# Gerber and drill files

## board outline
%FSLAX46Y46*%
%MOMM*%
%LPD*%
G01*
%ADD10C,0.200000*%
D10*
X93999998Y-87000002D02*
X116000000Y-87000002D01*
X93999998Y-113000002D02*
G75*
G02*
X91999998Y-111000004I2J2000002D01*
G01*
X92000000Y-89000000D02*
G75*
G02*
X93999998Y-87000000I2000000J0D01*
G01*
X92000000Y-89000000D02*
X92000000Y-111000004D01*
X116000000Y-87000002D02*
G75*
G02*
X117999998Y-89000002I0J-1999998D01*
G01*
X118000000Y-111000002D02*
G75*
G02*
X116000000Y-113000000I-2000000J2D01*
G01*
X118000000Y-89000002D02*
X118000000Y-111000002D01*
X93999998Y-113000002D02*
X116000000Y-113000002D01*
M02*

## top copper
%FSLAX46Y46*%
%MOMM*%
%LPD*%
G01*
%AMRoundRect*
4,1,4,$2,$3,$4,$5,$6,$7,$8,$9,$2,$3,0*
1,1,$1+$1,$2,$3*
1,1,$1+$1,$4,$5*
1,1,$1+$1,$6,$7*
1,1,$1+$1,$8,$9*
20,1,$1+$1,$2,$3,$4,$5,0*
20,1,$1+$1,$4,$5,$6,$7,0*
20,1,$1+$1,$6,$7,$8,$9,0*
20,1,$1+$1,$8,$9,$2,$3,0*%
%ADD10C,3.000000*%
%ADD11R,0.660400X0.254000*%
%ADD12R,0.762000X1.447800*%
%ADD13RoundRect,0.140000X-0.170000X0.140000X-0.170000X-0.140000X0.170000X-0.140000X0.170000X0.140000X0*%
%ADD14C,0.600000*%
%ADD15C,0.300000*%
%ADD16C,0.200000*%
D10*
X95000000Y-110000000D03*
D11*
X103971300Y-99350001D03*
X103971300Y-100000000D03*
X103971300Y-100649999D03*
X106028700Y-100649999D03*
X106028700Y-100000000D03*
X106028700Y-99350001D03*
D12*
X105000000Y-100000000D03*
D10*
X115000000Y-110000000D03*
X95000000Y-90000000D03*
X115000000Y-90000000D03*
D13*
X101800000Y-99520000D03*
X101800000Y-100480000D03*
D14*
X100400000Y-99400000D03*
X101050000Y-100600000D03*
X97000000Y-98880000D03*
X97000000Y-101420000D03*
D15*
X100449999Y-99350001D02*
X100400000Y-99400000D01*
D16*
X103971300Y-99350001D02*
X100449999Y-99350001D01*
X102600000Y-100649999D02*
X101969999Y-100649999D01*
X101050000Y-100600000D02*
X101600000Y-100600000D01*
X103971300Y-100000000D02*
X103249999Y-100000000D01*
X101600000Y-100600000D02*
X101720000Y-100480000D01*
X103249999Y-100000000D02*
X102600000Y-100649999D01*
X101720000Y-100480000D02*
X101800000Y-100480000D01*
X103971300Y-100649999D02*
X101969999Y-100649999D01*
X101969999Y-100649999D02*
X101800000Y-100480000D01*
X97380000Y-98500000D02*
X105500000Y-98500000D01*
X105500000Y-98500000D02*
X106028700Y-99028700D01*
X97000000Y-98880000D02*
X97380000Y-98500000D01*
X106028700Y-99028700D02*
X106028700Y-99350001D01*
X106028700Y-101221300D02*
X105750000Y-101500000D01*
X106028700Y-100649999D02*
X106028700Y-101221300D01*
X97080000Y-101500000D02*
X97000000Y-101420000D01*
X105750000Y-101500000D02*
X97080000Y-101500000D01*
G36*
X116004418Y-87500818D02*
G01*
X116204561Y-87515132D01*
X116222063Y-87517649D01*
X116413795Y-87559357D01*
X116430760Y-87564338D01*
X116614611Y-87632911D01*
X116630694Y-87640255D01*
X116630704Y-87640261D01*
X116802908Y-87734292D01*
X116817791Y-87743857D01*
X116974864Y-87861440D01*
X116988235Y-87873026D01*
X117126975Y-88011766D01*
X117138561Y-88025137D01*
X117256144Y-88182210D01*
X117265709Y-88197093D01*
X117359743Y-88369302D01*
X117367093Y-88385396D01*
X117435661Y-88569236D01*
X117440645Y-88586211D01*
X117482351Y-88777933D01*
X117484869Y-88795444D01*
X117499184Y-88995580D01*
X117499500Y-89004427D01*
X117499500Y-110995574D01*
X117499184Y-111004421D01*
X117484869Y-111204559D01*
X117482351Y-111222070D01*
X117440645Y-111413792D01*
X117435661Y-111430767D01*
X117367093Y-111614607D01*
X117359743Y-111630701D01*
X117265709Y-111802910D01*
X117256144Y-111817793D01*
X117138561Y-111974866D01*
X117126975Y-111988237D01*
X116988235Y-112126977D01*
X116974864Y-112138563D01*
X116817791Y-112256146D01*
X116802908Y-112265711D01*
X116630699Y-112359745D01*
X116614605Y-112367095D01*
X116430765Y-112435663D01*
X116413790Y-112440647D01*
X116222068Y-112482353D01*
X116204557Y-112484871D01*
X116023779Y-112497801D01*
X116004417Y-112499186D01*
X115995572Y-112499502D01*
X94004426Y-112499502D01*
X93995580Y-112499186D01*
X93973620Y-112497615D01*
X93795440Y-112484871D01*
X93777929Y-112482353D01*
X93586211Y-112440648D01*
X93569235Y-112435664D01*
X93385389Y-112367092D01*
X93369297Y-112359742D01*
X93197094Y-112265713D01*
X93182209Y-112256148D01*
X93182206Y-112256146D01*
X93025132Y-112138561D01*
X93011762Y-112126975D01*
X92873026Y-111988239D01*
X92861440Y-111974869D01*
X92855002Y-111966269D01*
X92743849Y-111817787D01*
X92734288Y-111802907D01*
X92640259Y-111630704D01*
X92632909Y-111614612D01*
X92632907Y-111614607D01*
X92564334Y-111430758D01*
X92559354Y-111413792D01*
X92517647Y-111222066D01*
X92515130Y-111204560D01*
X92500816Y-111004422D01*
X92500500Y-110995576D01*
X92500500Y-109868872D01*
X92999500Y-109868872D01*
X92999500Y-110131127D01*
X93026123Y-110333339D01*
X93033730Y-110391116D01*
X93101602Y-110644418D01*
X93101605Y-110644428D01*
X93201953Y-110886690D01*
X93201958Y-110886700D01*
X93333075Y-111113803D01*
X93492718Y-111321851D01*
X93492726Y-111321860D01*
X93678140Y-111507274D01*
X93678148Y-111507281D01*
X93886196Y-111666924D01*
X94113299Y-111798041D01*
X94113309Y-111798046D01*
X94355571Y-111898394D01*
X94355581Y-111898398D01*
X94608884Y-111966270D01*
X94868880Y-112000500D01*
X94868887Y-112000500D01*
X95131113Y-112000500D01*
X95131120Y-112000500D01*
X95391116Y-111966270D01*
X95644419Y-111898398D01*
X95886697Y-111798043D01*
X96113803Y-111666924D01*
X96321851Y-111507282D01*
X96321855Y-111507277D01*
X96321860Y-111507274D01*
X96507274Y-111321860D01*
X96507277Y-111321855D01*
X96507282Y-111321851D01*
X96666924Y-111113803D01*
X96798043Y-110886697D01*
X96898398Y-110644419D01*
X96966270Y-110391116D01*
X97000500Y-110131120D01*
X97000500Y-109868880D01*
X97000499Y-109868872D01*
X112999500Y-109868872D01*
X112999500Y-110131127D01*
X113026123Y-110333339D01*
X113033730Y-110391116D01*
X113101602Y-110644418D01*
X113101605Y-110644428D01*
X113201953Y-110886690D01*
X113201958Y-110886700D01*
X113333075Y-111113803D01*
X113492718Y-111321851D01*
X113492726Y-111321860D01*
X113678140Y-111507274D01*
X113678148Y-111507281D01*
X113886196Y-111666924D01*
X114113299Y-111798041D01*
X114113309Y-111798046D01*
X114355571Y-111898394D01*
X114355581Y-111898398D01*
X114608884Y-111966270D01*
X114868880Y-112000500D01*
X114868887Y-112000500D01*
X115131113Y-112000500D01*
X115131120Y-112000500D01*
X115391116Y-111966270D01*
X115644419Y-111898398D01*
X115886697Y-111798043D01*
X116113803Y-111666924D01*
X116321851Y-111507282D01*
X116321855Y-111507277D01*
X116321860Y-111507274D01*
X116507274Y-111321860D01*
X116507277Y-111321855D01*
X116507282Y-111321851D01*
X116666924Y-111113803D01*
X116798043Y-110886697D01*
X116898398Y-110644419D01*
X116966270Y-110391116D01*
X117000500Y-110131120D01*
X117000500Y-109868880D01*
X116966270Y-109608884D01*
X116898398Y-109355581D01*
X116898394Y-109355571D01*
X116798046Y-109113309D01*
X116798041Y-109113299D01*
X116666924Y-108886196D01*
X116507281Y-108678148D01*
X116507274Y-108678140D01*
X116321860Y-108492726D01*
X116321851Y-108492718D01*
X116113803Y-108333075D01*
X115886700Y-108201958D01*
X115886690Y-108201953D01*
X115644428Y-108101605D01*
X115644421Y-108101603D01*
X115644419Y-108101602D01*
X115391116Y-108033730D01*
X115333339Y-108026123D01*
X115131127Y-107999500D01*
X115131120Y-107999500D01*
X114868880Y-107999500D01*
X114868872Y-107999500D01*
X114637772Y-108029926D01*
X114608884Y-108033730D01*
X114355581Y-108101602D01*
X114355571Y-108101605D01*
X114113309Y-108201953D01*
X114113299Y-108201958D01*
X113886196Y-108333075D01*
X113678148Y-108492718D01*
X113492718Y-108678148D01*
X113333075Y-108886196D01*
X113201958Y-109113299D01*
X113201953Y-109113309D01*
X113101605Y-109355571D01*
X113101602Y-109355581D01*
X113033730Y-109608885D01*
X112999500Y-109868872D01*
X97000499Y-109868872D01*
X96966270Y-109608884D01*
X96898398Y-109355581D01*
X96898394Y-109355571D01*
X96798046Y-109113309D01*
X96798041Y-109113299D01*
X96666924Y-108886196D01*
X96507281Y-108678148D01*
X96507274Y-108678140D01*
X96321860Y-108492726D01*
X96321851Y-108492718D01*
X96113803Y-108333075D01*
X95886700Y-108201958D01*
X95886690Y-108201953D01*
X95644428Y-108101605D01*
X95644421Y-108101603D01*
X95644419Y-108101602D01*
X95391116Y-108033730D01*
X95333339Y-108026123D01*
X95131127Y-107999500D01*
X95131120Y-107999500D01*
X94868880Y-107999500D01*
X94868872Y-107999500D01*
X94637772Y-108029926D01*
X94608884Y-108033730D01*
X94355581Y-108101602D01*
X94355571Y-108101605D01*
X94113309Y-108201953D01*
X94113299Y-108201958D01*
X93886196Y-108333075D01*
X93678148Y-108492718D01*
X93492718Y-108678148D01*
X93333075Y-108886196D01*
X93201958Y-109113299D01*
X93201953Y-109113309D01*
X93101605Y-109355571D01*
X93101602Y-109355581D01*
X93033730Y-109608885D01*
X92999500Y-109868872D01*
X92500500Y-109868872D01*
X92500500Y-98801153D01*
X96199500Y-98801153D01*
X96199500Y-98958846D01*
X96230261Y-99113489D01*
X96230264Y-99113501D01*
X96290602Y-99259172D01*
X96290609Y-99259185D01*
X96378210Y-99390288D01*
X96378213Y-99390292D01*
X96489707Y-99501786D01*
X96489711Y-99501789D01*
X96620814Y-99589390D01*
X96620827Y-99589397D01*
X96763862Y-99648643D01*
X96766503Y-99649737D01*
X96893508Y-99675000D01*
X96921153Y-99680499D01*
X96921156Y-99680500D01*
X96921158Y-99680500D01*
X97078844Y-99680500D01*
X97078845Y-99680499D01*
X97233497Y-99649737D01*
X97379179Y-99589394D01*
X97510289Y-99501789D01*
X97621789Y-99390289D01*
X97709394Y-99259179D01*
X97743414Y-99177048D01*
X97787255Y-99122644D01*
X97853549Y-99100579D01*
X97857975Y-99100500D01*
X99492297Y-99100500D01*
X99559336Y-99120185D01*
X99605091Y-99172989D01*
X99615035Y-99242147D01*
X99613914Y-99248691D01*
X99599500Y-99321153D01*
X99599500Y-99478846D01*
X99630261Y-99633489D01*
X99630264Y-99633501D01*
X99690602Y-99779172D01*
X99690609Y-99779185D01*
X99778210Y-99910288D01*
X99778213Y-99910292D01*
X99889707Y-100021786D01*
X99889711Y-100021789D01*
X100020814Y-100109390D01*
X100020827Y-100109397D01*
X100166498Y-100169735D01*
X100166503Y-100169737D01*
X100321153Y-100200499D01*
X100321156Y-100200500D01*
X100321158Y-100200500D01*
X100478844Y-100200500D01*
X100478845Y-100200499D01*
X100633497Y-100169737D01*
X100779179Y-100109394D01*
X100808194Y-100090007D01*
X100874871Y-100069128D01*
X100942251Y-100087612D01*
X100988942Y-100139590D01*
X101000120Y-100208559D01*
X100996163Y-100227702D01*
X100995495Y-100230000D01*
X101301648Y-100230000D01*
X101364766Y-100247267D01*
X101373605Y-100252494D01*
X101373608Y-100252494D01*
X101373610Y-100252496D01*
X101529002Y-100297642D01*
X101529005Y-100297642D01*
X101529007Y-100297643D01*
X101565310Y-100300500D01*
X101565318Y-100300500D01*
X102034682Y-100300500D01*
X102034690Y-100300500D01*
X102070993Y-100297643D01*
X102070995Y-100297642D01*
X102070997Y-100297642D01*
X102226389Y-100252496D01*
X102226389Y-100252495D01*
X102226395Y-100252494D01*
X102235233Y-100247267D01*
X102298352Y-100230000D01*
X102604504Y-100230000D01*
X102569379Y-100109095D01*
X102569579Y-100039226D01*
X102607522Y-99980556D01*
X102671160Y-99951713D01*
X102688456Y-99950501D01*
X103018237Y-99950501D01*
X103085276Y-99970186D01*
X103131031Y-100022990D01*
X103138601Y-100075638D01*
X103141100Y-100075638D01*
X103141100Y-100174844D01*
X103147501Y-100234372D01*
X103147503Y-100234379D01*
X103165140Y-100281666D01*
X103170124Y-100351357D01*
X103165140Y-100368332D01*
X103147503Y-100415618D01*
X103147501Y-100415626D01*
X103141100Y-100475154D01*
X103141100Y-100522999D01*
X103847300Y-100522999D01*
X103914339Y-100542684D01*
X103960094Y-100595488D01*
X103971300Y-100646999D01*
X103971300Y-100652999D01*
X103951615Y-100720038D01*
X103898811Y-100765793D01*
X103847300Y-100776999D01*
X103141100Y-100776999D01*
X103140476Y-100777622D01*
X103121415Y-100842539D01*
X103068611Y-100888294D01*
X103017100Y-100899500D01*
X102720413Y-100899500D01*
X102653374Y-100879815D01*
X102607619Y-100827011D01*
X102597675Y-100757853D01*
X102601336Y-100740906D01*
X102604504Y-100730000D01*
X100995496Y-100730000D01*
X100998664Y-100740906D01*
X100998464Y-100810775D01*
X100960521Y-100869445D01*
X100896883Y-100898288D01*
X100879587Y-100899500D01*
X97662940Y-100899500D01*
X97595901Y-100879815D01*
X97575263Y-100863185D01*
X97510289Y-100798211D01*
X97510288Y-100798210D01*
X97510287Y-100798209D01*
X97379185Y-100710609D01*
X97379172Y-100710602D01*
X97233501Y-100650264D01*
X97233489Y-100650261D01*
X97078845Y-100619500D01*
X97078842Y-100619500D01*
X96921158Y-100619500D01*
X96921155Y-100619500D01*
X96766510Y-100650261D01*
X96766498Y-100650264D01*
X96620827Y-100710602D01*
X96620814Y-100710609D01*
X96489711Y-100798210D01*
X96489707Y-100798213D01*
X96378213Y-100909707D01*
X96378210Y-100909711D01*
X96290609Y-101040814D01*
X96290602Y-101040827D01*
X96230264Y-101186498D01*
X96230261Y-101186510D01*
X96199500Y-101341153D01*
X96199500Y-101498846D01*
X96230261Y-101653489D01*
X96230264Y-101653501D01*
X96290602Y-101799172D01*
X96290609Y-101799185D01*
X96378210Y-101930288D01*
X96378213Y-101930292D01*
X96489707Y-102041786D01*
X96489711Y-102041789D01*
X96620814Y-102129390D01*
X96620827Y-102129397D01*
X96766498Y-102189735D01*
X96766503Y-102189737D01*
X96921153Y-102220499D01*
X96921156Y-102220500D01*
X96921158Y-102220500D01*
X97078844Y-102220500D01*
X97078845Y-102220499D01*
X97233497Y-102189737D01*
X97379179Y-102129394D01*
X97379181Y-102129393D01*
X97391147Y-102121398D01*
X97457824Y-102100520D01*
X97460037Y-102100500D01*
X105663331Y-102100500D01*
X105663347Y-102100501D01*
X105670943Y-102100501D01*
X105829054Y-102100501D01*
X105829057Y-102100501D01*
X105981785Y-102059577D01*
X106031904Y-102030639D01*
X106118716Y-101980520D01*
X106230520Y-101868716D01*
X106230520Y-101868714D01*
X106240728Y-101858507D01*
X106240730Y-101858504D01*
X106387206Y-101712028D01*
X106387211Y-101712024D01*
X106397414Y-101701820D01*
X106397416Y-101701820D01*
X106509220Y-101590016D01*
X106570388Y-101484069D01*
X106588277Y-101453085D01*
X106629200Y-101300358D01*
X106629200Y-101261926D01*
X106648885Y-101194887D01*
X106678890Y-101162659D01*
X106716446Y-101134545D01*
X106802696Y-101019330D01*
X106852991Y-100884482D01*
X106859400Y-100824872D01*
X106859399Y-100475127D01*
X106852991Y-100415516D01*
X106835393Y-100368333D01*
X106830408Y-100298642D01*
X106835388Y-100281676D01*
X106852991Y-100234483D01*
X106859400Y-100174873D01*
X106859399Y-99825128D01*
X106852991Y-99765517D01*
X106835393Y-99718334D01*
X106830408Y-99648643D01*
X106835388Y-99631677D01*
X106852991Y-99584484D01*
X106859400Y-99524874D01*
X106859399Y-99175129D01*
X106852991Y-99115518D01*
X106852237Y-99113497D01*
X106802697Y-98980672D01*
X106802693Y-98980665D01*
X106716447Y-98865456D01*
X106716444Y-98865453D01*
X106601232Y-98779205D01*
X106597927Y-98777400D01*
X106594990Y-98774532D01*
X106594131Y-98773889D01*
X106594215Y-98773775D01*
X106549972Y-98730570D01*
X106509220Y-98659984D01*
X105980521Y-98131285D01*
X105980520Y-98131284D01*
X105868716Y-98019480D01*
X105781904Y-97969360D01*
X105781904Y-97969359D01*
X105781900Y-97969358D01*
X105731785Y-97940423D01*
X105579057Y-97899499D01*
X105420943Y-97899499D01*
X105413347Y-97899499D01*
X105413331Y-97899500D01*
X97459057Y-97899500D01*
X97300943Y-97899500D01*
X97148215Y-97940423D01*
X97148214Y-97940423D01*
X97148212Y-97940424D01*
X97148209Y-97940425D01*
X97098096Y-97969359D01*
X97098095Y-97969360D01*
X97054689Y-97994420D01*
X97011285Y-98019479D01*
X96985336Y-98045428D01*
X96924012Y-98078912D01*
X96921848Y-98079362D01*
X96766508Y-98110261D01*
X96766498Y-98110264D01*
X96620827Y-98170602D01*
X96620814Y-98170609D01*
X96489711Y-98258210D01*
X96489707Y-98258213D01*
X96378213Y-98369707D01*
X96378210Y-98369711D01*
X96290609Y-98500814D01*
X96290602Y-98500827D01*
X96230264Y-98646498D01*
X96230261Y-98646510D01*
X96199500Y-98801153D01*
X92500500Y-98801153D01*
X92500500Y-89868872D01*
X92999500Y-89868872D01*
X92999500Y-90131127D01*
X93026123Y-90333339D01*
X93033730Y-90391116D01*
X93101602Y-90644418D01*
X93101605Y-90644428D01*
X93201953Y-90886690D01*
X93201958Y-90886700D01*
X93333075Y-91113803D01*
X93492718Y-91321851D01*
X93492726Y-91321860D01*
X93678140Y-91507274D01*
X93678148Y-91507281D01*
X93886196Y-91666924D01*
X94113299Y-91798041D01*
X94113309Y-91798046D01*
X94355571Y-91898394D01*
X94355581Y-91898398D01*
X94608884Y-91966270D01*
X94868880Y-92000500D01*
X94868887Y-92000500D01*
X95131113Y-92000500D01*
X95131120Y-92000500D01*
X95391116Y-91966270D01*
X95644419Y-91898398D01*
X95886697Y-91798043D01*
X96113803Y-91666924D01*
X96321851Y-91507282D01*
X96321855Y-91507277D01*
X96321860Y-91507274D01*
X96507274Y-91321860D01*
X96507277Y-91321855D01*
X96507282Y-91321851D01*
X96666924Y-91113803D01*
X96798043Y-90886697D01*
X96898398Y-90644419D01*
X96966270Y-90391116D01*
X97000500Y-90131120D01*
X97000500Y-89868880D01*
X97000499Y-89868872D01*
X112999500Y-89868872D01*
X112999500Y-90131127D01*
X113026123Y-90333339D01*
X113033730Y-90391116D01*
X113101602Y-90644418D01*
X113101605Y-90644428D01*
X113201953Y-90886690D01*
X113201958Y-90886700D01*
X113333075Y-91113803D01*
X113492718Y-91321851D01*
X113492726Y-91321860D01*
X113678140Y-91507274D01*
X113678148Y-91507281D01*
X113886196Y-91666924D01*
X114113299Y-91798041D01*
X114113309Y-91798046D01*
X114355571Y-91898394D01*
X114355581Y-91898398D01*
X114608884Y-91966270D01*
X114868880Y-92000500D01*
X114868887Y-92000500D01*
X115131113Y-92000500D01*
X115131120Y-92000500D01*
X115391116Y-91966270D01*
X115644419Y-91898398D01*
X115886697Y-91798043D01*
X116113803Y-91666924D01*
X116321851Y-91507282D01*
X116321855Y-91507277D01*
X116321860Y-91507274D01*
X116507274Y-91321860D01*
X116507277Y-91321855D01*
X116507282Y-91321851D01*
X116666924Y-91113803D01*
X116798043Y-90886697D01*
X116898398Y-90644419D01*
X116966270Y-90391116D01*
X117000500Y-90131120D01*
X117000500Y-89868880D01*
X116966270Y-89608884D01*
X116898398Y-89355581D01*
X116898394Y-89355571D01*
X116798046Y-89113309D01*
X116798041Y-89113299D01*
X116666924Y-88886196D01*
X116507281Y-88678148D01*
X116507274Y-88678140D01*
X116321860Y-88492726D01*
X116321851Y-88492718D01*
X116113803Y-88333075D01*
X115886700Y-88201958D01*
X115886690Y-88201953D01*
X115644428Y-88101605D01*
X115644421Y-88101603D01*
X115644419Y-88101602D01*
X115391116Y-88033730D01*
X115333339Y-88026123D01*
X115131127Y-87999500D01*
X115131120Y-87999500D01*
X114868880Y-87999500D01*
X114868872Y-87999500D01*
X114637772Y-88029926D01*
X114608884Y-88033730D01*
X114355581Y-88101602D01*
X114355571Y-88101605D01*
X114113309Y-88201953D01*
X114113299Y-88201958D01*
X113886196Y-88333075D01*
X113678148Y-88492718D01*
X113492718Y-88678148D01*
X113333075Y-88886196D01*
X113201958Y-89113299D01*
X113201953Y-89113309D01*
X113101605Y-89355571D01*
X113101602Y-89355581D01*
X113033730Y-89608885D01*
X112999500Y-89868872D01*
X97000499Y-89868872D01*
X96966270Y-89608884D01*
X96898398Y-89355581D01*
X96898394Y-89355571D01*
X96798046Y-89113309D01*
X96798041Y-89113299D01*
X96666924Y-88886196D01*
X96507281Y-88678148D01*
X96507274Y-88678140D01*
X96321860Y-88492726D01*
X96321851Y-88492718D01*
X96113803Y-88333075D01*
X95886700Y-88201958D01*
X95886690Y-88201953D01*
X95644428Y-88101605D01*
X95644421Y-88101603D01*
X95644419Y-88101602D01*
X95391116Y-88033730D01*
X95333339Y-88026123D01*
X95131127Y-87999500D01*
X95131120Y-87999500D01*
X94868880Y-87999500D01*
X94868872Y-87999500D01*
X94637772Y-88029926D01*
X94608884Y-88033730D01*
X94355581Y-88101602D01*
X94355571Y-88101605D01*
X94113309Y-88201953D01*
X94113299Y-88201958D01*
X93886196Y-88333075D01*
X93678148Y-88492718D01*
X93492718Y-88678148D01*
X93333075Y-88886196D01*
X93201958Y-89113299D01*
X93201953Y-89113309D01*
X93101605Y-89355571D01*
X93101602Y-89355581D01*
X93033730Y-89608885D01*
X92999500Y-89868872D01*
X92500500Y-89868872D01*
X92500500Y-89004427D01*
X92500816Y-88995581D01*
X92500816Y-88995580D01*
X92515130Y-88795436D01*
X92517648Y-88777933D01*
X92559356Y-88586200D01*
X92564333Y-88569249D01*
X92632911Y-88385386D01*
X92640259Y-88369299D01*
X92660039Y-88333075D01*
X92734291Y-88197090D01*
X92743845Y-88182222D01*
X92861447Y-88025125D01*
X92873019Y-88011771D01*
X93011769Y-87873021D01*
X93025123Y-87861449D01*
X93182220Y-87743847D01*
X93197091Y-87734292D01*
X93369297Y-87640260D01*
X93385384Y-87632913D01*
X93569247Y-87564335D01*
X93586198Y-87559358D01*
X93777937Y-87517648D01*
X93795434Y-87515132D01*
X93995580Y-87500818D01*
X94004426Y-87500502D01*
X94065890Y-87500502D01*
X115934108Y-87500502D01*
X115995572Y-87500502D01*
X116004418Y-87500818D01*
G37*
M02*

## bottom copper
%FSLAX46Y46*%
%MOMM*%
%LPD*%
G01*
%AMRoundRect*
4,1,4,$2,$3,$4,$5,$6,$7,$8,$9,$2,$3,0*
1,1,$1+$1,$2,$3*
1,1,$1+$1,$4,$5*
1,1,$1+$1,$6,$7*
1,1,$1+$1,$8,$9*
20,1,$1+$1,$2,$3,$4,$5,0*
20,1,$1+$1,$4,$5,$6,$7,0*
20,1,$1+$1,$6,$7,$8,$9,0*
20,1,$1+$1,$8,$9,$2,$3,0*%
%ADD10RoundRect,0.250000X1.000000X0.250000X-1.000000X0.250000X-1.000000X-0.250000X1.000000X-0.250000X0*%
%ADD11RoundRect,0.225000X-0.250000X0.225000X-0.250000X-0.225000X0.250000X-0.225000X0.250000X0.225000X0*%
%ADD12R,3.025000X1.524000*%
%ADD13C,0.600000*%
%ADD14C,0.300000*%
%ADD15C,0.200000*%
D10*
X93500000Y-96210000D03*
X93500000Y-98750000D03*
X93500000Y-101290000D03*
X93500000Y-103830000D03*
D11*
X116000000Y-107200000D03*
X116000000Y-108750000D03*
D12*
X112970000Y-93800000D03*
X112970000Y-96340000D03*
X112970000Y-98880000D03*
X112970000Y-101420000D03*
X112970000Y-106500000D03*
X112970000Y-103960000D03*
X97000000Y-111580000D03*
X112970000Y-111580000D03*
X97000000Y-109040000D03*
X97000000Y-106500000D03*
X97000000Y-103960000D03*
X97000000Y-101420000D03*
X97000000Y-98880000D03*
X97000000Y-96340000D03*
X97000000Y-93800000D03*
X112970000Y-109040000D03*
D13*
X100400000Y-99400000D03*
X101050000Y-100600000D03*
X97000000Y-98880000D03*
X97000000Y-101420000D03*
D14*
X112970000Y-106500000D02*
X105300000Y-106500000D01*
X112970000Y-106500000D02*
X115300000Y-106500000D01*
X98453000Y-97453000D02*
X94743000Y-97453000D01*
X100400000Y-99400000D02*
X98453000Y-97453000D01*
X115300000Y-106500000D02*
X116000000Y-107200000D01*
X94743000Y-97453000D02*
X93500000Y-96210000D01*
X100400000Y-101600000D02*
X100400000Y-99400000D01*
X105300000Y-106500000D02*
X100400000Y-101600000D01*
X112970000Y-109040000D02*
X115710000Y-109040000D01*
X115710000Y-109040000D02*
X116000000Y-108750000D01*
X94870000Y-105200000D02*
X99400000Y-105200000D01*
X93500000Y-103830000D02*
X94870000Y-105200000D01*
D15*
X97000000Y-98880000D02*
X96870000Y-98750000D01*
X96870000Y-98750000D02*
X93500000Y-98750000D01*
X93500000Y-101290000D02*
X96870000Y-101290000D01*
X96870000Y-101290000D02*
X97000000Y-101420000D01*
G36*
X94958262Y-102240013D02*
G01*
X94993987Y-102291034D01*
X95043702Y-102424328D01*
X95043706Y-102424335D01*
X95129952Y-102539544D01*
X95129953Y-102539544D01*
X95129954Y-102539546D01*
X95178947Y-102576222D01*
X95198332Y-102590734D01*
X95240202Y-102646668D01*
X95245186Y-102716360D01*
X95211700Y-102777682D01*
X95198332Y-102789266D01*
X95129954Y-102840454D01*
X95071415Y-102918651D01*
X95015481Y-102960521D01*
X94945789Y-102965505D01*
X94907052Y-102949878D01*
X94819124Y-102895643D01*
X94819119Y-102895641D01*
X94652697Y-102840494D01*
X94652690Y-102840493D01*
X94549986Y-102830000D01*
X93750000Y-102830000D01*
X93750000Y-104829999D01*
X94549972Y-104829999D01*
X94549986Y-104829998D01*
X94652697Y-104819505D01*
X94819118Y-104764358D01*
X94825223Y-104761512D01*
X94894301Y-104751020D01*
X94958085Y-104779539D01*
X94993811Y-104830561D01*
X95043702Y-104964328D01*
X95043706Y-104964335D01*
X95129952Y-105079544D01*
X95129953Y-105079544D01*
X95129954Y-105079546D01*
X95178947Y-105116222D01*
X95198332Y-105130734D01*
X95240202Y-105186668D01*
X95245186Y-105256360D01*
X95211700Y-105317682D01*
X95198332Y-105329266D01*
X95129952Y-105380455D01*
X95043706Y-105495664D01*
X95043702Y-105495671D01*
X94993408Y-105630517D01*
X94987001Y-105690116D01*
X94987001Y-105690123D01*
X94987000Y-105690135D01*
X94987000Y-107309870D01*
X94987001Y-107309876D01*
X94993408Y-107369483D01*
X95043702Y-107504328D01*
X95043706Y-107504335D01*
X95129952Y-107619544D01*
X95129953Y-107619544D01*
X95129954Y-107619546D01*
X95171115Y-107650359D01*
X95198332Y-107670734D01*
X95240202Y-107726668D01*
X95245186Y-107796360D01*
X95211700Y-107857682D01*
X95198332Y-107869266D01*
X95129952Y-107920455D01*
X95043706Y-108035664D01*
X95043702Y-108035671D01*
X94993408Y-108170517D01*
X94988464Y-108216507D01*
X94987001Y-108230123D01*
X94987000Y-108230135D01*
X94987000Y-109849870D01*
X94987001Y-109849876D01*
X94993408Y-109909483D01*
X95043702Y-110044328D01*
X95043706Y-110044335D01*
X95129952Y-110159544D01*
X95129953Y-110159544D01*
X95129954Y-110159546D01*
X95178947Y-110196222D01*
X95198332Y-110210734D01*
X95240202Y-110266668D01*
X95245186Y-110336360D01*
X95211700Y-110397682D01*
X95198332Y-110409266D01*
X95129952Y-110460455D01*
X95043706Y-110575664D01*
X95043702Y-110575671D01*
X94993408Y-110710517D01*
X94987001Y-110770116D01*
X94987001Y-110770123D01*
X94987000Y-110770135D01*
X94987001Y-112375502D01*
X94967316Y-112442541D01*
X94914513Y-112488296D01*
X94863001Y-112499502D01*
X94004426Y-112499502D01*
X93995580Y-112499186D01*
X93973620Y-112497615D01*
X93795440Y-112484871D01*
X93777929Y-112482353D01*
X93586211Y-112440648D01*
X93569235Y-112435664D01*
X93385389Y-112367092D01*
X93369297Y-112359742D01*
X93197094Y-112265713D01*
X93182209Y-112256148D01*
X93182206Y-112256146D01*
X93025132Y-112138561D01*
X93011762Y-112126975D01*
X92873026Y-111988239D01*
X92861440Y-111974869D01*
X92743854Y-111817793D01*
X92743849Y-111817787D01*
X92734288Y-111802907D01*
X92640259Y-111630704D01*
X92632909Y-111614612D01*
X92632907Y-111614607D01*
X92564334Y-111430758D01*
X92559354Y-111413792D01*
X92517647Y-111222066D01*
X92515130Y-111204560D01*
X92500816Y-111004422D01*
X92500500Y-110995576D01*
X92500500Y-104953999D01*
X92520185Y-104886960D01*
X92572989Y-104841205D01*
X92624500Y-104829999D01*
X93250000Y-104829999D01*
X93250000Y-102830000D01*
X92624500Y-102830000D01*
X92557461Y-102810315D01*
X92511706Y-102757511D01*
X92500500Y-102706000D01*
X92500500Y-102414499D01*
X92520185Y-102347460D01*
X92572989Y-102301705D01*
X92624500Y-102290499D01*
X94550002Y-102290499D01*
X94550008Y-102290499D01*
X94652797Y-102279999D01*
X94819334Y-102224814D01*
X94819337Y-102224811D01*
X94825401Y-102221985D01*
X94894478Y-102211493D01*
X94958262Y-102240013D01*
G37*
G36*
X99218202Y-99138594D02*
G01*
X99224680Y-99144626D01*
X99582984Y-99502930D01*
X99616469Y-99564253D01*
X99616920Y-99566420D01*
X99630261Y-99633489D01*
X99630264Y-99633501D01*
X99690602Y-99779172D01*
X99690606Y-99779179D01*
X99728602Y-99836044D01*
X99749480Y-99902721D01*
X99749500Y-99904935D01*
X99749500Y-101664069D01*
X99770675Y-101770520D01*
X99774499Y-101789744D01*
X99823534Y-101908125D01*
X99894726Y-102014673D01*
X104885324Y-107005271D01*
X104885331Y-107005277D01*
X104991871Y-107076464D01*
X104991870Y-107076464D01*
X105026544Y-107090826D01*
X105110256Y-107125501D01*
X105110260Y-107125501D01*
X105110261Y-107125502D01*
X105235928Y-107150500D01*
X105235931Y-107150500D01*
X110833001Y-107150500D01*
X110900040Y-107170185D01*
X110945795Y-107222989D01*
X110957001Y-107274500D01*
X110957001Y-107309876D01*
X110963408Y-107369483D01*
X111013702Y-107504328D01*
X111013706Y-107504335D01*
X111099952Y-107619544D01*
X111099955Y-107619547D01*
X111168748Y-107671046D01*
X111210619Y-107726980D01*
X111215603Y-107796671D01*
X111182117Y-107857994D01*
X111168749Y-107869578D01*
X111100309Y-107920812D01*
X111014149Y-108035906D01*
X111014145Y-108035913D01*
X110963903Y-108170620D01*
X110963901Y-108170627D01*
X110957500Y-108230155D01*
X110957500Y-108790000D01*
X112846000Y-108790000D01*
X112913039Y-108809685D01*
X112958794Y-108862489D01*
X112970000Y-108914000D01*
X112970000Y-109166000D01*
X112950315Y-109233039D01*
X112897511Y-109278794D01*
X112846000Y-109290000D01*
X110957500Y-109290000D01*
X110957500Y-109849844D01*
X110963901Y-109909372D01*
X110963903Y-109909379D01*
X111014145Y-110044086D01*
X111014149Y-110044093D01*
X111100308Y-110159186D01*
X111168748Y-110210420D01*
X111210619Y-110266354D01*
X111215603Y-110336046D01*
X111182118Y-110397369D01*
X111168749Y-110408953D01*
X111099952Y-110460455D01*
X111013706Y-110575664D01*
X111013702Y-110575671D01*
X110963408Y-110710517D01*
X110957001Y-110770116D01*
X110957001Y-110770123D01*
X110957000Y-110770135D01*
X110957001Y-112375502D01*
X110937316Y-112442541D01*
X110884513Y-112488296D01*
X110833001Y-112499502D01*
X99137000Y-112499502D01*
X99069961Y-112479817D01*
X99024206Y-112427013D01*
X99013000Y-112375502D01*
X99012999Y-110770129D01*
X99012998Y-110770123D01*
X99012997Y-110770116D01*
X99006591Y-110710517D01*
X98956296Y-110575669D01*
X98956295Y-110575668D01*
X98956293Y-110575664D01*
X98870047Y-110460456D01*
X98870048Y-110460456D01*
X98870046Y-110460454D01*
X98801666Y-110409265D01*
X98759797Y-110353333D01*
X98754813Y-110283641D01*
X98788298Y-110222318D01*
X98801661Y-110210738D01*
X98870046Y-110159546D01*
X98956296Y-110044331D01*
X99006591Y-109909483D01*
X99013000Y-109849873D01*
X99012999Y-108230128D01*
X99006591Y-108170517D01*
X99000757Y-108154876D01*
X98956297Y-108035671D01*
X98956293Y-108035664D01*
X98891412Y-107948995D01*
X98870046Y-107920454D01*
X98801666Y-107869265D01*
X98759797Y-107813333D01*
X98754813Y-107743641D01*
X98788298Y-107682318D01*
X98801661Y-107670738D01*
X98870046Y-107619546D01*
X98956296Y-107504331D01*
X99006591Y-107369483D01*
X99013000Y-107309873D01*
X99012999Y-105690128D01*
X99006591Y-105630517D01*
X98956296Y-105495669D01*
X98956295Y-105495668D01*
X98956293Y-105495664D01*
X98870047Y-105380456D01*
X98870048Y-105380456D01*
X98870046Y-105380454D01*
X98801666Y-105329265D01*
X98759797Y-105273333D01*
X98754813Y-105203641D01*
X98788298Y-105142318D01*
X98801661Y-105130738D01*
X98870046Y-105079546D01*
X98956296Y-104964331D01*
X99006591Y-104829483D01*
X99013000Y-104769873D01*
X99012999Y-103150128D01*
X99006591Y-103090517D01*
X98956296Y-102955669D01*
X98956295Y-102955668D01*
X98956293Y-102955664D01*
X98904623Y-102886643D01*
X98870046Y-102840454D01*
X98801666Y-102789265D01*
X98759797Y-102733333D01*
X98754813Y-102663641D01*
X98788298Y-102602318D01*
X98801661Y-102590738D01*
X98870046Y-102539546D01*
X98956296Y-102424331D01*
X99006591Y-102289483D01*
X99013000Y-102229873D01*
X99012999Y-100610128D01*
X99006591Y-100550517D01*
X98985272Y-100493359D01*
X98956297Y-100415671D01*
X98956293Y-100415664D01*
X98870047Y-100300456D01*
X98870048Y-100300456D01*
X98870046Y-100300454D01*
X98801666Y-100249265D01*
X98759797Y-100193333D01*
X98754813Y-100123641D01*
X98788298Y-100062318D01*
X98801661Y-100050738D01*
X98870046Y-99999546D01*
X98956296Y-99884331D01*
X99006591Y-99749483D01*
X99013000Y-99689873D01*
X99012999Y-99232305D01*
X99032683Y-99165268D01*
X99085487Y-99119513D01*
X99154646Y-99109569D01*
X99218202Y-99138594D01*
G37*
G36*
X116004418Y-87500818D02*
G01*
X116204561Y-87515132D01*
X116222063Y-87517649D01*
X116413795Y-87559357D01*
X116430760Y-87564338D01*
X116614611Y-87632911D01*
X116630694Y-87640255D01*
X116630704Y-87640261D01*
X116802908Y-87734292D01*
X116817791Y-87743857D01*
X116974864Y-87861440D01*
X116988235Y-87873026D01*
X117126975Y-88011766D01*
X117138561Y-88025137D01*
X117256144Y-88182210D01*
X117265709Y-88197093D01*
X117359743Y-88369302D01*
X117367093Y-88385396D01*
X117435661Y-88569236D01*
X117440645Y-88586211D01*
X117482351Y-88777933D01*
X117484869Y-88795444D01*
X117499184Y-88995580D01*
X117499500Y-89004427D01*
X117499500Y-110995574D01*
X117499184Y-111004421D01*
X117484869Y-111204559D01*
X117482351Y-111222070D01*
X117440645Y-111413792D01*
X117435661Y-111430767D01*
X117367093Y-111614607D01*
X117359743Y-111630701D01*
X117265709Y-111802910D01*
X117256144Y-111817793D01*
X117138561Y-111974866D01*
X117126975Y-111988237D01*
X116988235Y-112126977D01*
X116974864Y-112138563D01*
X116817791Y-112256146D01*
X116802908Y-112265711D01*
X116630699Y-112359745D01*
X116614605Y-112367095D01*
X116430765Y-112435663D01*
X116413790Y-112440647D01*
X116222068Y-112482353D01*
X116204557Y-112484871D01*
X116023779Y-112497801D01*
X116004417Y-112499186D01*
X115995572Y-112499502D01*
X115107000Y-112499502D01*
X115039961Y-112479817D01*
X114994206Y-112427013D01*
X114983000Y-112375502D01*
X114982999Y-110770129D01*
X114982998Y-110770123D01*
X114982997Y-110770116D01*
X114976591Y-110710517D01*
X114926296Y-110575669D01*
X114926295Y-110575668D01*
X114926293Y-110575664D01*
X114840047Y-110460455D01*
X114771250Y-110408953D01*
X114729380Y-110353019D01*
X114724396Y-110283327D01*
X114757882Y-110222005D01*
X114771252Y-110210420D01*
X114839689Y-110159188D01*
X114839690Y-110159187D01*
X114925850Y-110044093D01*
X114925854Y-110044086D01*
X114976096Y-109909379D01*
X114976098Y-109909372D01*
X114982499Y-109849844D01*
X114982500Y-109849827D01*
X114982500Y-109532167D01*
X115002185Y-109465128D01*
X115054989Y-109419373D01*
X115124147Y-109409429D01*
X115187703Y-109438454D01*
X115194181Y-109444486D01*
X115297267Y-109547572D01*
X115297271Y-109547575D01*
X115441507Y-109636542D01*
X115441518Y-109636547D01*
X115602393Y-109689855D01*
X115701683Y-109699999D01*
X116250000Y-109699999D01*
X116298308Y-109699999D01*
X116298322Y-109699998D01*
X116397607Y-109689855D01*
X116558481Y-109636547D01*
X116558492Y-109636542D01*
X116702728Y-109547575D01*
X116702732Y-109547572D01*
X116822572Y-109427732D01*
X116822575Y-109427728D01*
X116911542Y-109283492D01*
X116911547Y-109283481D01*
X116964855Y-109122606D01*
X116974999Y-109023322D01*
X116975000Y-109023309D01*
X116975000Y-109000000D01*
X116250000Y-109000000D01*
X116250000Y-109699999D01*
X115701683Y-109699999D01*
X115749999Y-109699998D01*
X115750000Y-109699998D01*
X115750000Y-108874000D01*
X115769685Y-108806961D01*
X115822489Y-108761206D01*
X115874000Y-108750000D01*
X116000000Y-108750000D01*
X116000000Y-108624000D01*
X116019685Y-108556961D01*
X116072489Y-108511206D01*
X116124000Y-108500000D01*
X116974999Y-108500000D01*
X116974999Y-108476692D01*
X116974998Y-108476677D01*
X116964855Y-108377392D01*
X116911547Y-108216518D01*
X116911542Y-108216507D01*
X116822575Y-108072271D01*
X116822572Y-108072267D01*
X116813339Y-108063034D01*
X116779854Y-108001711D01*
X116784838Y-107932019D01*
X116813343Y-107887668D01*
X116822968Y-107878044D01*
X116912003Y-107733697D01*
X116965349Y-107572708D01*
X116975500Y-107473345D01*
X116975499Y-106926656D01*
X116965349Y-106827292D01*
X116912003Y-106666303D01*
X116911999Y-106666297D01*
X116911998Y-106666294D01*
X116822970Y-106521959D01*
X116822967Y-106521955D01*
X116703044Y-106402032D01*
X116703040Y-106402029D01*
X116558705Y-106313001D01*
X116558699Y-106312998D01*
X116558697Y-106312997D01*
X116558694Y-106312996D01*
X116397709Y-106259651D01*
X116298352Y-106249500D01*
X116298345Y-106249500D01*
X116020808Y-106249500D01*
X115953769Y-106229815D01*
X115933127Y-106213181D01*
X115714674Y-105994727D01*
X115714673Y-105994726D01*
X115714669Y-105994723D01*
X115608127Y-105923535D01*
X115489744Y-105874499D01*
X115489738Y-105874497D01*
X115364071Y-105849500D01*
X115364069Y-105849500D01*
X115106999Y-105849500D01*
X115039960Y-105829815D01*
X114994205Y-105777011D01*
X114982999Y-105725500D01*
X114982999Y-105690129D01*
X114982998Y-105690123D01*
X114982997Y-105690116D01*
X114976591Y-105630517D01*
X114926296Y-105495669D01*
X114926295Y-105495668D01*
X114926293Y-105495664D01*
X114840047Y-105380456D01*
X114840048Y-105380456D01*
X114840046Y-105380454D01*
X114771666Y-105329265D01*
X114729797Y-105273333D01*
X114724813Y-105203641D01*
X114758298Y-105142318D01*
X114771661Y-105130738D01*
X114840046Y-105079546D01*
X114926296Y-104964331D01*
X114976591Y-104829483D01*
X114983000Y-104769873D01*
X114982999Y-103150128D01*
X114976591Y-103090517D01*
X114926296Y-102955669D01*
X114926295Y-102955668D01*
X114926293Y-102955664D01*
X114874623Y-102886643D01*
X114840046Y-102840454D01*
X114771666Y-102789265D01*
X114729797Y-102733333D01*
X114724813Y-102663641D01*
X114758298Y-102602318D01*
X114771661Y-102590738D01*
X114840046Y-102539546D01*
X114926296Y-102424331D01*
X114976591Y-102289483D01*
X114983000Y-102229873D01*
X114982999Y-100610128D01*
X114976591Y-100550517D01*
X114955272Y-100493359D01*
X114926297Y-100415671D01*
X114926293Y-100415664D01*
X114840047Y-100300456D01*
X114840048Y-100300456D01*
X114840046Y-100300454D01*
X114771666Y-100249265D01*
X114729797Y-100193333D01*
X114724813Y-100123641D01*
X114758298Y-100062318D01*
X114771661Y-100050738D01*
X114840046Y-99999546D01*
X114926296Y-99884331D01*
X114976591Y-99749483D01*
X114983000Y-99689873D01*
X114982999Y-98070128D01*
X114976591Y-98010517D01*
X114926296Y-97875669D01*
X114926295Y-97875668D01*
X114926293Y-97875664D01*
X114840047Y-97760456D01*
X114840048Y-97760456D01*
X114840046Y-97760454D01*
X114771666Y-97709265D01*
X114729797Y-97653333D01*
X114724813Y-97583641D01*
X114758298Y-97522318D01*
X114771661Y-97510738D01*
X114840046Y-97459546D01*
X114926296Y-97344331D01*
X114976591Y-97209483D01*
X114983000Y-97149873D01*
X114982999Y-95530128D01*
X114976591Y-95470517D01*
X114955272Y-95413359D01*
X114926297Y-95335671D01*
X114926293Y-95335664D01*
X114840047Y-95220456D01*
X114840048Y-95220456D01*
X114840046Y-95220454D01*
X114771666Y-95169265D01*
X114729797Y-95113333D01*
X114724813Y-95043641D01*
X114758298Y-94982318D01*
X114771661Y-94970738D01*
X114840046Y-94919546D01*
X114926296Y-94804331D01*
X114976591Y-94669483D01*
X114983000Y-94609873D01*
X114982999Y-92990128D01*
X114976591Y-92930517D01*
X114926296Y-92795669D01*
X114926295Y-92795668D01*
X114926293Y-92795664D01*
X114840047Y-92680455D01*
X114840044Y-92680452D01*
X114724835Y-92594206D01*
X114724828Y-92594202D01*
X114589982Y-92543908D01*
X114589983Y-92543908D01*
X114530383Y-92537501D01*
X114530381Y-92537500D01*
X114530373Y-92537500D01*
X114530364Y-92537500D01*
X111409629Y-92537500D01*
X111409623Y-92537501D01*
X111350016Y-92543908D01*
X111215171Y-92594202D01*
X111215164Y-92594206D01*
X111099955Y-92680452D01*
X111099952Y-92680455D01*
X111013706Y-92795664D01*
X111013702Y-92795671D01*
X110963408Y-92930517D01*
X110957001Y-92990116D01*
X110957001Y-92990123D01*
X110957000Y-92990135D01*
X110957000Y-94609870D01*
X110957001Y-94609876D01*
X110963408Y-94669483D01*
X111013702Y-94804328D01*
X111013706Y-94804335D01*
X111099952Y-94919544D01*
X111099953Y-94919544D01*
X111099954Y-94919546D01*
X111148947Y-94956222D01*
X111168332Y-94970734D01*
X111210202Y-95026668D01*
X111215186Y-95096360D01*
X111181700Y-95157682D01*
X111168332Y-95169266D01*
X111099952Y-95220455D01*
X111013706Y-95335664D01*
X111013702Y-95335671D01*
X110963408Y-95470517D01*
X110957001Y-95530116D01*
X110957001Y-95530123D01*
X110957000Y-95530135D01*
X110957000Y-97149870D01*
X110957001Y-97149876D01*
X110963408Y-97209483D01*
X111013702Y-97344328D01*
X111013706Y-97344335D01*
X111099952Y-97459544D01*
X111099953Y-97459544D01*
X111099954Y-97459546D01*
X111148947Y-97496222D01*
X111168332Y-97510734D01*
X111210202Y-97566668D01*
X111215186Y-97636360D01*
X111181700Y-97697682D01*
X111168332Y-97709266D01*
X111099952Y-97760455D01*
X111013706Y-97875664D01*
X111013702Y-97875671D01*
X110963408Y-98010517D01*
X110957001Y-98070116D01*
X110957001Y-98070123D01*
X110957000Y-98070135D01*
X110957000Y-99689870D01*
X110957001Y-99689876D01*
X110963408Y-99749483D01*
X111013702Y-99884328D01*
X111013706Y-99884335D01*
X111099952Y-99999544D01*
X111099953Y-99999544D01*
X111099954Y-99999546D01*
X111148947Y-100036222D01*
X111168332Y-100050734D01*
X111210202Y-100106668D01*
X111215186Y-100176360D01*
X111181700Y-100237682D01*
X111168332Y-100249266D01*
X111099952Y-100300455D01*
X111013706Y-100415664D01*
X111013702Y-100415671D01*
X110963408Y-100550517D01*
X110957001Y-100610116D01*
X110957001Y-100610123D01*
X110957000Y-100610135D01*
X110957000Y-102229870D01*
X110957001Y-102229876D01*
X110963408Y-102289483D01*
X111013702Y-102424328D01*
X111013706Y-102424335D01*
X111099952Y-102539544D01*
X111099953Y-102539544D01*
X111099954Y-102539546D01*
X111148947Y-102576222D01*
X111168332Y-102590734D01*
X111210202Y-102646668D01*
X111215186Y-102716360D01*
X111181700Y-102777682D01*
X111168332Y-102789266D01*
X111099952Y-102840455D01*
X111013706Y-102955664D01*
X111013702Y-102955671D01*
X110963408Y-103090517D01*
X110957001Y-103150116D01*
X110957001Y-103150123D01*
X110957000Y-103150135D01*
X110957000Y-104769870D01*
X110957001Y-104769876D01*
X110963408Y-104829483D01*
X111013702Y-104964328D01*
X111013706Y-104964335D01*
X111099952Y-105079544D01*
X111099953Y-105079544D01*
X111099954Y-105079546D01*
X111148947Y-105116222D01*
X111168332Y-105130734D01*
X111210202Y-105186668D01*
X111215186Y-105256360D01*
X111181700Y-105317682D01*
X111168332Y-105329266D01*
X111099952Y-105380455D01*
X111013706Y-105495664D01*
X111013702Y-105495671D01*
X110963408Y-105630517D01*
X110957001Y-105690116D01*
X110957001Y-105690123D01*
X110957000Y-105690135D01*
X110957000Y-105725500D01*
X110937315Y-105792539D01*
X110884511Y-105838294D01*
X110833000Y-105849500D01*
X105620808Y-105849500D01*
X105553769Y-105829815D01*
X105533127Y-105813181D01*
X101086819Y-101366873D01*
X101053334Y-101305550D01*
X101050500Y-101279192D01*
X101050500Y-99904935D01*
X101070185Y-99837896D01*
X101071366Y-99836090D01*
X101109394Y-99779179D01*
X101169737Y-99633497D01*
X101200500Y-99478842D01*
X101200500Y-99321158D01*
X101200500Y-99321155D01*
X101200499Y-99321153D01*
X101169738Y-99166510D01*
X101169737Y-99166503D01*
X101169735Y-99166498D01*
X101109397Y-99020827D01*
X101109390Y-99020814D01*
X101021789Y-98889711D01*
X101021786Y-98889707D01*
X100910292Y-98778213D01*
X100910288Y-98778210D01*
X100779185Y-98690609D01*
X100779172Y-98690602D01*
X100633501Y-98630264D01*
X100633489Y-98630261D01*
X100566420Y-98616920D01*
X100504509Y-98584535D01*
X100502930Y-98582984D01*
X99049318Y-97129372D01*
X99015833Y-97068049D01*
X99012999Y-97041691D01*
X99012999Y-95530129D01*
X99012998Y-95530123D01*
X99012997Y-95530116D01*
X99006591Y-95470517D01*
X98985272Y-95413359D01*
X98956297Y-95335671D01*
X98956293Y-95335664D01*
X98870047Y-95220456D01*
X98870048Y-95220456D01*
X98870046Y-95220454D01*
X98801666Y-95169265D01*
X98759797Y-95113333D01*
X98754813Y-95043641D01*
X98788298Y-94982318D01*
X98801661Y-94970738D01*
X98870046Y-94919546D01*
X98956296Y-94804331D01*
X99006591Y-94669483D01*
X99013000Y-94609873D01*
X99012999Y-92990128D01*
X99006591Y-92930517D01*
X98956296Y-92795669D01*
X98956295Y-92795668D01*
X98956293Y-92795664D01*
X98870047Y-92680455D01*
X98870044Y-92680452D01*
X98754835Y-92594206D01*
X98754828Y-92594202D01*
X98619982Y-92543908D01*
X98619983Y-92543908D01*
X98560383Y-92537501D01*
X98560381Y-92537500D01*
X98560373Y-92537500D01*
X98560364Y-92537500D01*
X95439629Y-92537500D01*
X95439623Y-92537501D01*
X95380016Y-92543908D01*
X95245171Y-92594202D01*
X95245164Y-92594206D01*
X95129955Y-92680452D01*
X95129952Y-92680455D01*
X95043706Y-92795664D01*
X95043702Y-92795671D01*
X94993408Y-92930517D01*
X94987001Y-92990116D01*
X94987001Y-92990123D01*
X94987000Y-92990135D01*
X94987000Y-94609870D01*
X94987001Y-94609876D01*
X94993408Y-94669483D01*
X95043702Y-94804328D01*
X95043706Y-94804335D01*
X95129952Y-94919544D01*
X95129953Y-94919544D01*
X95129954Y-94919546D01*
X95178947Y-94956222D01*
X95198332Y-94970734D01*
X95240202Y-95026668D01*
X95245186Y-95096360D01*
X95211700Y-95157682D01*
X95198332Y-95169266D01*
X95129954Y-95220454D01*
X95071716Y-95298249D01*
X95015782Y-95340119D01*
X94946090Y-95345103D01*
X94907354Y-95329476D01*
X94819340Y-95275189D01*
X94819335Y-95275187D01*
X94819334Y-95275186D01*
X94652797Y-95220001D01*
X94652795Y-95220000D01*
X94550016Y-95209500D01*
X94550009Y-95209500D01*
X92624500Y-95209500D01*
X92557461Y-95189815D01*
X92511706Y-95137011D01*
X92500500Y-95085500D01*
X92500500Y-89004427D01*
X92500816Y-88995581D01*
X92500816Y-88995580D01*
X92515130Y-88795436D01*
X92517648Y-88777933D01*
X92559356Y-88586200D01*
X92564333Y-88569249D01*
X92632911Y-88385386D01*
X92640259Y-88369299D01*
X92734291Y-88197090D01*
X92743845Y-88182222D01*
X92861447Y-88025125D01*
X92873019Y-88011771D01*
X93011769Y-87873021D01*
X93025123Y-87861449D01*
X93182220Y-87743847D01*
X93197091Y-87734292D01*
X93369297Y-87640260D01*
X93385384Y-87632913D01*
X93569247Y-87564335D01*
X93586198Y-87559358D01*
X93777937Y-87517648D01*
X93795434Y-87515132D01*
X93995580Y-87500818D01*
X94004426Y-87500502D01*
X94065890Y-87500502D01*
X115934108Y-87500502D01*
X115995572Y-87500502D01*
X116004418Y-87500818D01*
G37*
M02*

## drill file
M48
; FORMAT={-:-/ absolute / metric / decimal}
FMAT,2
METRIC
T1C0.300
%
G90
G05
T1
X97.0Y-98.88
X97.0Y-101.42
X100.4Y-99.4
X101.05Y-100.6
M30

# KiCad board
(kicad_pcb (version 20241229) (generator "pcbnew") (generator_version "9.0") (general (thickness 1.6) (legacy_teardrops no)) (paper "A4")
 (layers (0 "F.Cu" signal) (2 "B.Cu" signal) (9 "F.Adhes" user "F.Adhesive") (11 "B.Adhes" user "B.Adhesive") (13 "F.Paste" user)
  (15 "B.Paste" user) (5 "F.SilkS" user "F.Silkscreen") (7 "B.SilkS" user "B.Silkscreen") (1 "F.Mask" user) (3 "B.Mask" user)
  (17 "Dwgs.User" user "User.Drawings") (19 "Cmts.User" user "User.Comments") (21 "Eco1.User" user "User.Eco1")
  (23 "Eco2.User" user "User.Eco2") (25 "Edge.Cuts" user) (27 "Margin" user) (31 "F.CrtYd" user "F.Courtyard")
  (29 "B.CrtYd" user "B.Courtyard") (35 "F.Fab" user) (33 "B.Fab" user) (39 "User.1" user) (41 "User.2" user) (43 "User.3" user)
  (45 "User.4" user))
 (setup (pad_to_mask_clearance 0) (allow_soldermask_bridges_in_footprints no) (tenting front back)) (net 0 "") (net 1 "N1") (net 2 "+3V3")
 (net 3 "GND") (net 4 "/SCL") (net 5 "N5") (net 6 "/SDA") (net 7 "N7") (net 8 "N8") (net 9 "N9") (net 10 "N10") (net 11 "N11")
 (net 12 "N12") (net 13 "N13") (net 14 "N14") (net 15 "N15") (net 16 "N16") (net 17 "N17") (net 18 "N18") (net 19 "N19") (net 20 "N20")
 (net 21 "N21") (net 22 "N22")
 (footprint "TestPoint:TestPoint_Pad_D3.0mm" (layer "F.Cu") (at 95 110)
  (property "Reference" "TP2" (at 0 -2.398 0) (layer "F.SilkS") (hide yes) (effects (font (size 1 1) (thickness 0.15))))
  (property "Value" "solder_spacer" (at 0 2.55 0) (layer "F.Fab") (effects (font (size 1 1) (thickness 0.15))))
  (pad "1" smd circle (at 0 0) (size 3 3) (layers "F.Cu" "F.Mask") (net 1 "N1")))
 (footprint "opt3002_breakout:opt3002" (layer "F.Cu") (at 105 100)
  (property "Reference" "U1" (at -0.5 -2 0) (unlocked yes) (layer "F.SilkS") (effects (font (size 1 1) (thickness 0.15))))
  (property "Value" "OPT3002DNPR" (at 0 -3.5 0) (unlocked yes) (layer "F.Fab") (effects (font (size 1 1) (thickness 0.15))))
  (pad "1" smd rect (at -1.0287 -0.649999) (size 0.6604 0.254) (layers "F.Cu" "F.Mask" "F.Paste") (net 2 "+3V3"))
  (pad "2" smd rect (at -1.0287 0) (size 0.6604 0.254) (layers "F.Cu" "F.Mask" "F.Paste") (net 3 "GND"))
  (pad "3" smd rect (at -1.0287 0.649999) (size 0.6604 0.254) (layers "F.Cu" "F.Mask" "F.Paste") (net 3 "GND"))
  (pad "4" smd rect (at 1.0287 0.649999) (size 0.6604 0.254) (layers "F.Cu" "F.Mask" "F.Paste") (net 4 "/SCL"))
  (pad "5" smd rect (at 1.0287 0) (size 0.6604 0.254) (layers "F.Cu" "F.Mask" "F.Paste") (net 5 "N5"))
  (pad "6" smd rect (at 1.0287 -0.649999) (size 0.6604 0.254) (layers "F.Cu" "F.Mask" "F.Paste") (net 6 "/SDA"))
  (pad "7" smd rect (at 0 0) (size 0.762 1.4478) (layers "F.Cu" "F.Mask" "F.Paste") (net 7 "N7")))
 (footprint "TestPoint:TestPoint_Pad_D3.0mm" (layer "F.Cu") (at 115 110)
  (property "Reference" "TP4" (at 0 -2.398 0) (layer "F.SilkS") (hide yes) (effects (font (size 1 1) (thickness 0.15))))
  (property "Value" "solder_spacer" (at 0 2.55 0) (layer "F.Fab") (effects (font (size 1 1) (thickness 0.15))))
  (pad "1" smd circle (at 0 0) (size 3 3) (layers "F.Cu" "F.Mask") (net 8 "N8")))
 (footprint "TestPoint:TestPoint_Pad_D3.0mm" (layer "F.Cu") (at 95 90)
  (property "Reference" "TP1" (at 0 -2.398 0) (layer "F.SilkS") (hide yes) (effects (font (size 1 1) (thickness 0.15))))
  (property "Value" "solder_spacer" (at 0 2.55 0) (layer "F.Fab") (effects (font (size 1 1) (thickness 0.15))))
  (pad "1" smd circle (at 0 0) (size 3 3) (layers "F.Cu" "F.Mask") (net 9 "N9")))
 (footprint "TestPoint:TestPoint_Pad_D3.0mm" (layer "F.Cu") (at 115 90)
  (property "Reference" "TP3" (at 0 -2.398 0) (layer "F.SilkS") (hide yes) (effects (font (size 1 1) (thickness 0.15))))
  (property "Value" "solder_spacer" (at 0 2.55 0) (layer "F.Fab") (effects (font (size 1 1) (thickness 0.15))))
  (pad "1" smd circle (at 0 0) (size 3 3) (layers "F.Cu" "F.Mask") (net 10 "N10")))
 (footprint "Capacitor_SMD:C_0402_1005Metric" (layer "F.Cu") (at 101.8 100 -90)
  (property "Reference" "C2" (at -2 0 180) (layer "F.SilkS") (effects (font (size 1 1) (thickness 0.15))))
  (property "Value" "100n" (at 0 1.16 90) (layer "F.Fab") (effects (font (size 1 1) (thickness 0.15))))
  (pad "1" smd roundrect (at -0.48 0 270) (size 0.56 0.62) (layers "F.Cu" "F.Mask" "F.Paste") (roundrect_rratio 0.25) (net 2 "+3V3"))
  (pad "2" smd roundrect (at 0.48 0 270) (size 0.56 0.62) (layers "F.Cu" "F.Mask" "F.Paste") (roundrect_rratio 0.25) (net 3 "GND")))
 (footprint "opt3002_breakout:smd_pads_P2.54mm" (layer "B.Cu") (at 93.5 100.02 180)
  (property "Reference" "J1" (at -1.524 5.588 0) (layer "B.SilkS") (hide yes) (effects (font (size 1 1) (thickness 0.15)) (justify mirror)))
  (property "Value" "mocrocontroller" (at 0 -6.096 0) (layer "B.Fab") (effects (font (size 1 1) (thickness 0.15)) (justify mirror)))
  (pad "1" smd roundrect (at 0 3.81 180) (size 2.5 1) (layers "B.Cu" "B.Mask" "B.Paste") (roundrect_rratio 0.25) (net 2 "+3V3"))
  (pad "2" smd roundrect (at 0 1.27 180) (size 2.5 1) (layers "B.Cu" "B.Mask" "B.Paste") (roundrect_rratio 0.25) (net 6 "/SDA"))
  (pad "3" smd roundrect (at 0 -1.27 180) (size 2.5 1) (layers "B.Cu" "B.Mask" "B.Paste") (roundrect_rratio 0.25) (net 4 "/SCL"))
  (pad "4" smd roundrect (at 0 -3.81 180) (size 2.5 1) (layers "B.Cu" "B.Mask" "B.Paste") (roundrect_rratio 0.25) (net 3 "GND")))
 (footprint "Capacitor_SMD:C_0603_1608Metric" (layer "B.Cu") (at 116 107.975 -90)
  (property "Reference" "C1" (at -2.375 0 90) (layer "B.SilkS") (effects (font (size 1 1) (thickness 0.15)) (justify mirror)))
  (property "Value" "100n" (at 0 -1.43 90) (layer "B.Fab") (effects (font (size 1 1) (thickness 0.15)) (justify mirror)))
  (pad "1" smd roundrect (at -0.775 0 270) (size 0.9 0.95) (layers "B.Cu" "B.Mask" "B.Paste") (roundrect_rratio 0.25) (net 2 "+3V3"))
  (pad "2" smd roundrect (at 0.775 0 270) (size 0.9 0.95) (layers "B.Cu" "B.Mask" "B.Paste") (roundrect_rratio 0.25) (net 3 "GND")))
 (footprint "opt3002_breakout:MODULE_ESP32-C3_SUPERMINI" (layer "B.Cu") (at 104.985 101.68)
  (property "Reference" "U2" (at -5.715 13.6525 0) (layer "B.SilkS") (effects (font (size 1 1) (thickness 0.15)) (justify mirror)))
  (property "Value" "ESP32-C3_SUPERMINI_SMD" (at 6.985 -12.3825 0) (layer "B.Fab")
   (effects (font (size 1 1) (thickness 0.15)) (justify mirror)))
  (pad "0" smd rect (at 7.985 -7.88) (size 3.025 1.524) (layers "B.Cu" "B.Mask" "B.Paste") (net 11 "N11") (solder_mask_margin 0.102))
  (pad "1" smd rect (at 7.985 -5.34) (size 3.025 1.524) (layers "B.Cu" "B.Mask" "B.Paste") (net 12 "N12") (solder_mask_margin 0.102))
  (pad "2" smd rect (at 7.985 -2.8) (size 3.025 1.524) (layers "B.Cu" "B.Mask" "B.Paste") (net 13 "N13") (solder_mask_margin 0.102))
  (pad "3" smd rect (at 7.985 -0.26) (size 3.025 1.524) (layers "B.Cu" "B.Mask" "B.Paste") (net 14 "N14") (solder_mask_margin 0.102))
  (pad "3.3" smd rect (at 7.985 4.82) (size 3.025 1.524) (layers "B.Cu" "B.Mask" "B.Paste") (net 2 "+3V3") (solder_mask_margin 0.102))
  (pad "4" smd rect (at 7.985 2.28) (size 3.025 1.524) (layers "B.Cu" "B.Mask" "B.Paste") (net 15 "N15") (solder_mask_margin 0.102))
  (pad "5" smd rect (at -7.985 9.9) (size 3.025 1.524) (layers "B.Cu" "B.Mask" "B.Paste") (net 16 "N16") (solder_mask_margin 0.102))
  (pad "5V" smd rect (at 7.985 9.9) (size 3.025 1.524) (layers "B.Cu" "B.Mask" "B.Paste") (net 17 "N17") (solder_mask_margin 0.102))
  (pad "6" smd rect (at -7.985 7.36) (size 3.025 1.524) (layers "B.Cu" "B.Mask" "B.Paste") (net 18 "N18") (solder_mask_margin 0.102))
  (pad "7" smd rect (at -7.985 4.82) (size 3.025 1.524) (layers "B.Cu" "B.Mask" "B.Paste") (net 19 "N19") (solder_mask_margin 0.102))
  (pad "8" smd rect (at -7.985 2.28) (size 3.025 1.524) (layers "B.Cu" "B.Mask" "B.Paste") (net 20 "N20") (solder_mask_margin 0.102))
  (pad "9" smd rect (at -7.985 -0.26) (size 3.025 1.524) (layers "B.Cu" "B.Mask" "B.Paste") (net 4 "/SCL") (solder_mask_margin 0.102))
  (pad "10" smd rect (at -7.985 -2.8) (size 3.025 1.524) (layers "B.Cu" "B.Mask" "B.Paste") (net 6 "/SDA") (solder_mask_margin 0.102))
  (pad "20" smd rect (at -7.985 -5.34) (size 3.025 1.524) (layers "B.Cu" "B.Mask" "B.Paste") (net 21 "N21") (solder_mask_margin 0.102))
  (pad "21" smd rect (at -7.985 -7.88) (size 3.025 1.524) (layers "B.Cu" "B.Mask" "B.Paste") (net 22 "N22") (solder_mask_margin 0.102))
  (pad "G" smd rect (at 7.985 7.36) (size 3.025 1.524) (layers "B.Cu" "B.Mask" "B.Paste") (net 3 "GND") (solder_mask_margin 0.102)))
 (gr_line (start 93.999998 87.000002) (end 116 87.000002) (stroke (width 0.2) (type default)) (layer "Edge.Cuts"))
 (gr_arc (start 93.999998 113.000002) (mid 92.585786 112.414216) (end 92 111.000004) (stroke (width 0.2) (type default)) (layer "Edge.Cuts"))
 (gr_arc (start 92 89) (mid 92.585786 87.585788) (end 93.999998 87.000002) (stroke (width 0.2) (type default)) (layer "Edge.Cuts"))
 (gr_line (start 92 89) (end 92 111.000004) (stroke (width 0.2) (type default)) (layer "Edge.Cuts"))
 (gr_arc (start 116 87.000002) (mid 117.414214 87.585788) (end 118 89.000002) (stroke (width 0.2) (type default)) (layer "Edge.Cuts"))
 (gr_arc (start 118 111.000002) (mid 117.414214 112.414216) (end 116 113.000002) (stroke (width 0.2) (type default)) (layer "Edge.Cuts"))
 (gr_line (start 118 89.000002) (end 118 111.000002) (stroke (width 0.2) (type default)) (layer "Edge.Cuts"))
 (gr_line (start 93.999998 113.000002) (end 116 113.000002) (stroke (width 0.2) (type default)) (layer "Edge.Cuts"))
 (segment (start 100.449999 99.350001) (end 100.4 99.4) (width 0.3) (layer "F.Cu") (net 2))
 (segment (start 103.9713 99.350001) (end 100.449999 99.350001) (width 0.2) (layer "F.Cu") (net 2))
 (via (at 100.4 99.4) (size 0.6) (drill 0.3) (layers "F.Cu" "B.Cu") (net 2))
 (segment (start 112.97 106.5) (end 105.3 106.5) (width 0.3) (layer "B.Cu") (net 2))
 (segment (start 112.97 106.5) (end 115.3 106.5) (width 0.3) (layer "B.Cu") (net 2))
 (segment (start 98.453 97.453) (end 94.743 97.453) (width 0.3) (layer "B.Cu") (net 2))
 (segment (start 100.4 99.4) (end 98.453 97.453) (width 0.3) (layer "B.Cu") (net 2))
 (segment (start 115.3 106.5) (end 116 107.2) (width 0.3) (layer "B.Cu") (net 2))
 (segment (start 94.743 97.453) (end 93.5 96.21) (width 0.3) (layer "B.Cu") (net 2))
 (segment (start 100.4 101.6) (end 100.4 99.4) (width 0.3) (layer "B.Cu") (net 2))
 (segment (start 105.3 106.5) (end 100.4 101.6) (width 0.3) (layer "B.Cu") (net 2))
 (segment (start 102.6 100.649999) (end 101.969999 100.649999) (width 0.2) (layer "F.Cu") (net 3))
 (segment (start 101.05 100.6) (end 101.6 100.6) (width 0.2) (layer "F.Cu") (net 3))
 (segment (start 103.9713 100) (end 103.249999 100) (width 0.2) (layer "F.Cu") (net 3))
 (segment (start 101.6 100.6) (end 101.72 100.48) (width 0.2) (layer "F.Cu") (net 3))
 (segment (start 103.249999 100) (end 102.6 100.649999) (width 0.2) (layer "F.Cu") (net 3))
 (segment (start 101.72 100.48) (end 101.8 100.48) (width 0.2) (layer "F.Cu") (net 3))
 (segment (start 103.9713 100.649999) (end 101.969999 100.649999) (width 0.2) (layer "F.Cu") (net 3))
 (segment (start 101.969999 100.649999) (end 101.8 100.48) (width 0.2) (layer "F.Cu") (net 3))
 (via (at 101.05 100.6) (size 0.6) (drill 0.3) (layers "F.Cu" "B.Cu") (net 3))
 (segment (start 112.97 109.04) (end 115.71 109.04) (width 0.3) (layer "B.Cu") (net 3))
 (segment (start 115.71 109.04) (end 116 108.75) (width 0.3) (layer "B.Cu") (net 3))
 (segment (start 94.87 105.2) (end 99.4 105.2) (width 0.3) (layer "B.Cu") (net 3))
 (segment (start 93.5 103.83) (end 94.87 105.2) (width 0.3) (layer "B.Cu") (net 3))
 (segment (start 97.38 98.5) (end 105.5 98.5) (width 0.2) (layer "F.Cu") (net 6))
 (segment (start 105.5 98.5) (end 106.0287 99.0287) (width 0.2) (layer "F.Cu") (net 6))
 (segment (start 97 98.88) (end 97.38 98.5) (width 0.2) (layer "F.Cu") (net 6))
 (segment (start 106.0287 99.0287) (end 106.0287 99.350001) (width 0.2) (layer "F.Cu") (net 6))
 (via (at 97 98.88) (size 0.6) (drill 0.3) (layers "F.Cu" "B.Cu") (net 6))
 (segment (start 97 98.88) (end 96.87 98.75) (width 0.2) (layer "B.Cu") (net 6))
 (segment (start 96.87 98.75) (end 93.5 98.75) (width 0.2) (layer "B.Cu") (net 6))
 (segment (start 106.0287 101.2213) (end 105.75 101.5) (width 0.2) (layer "F.Cu") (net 4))
 (segment (start 106.0287 100.649999) (end 106.0287 101.2213) (width 0.2) (layer "F.Cu") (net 4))
 (segment (start 97.08 101.5) (end 97 101.42) (width 0.2) (layer "F.Cu") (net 4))
 (segment (start 105.75 101.5) (end 97.08 101.5) (width 0.2) (layer "F.Cu") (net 4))
 (via (at 97 101.42) (size 0.6) (drill 0.3) (layers "F.Cu" "B.Cu") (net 4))
 (segment (start 93.5 101.29) (end 96.87 101.29) (width 0.2) (layer "B.Cu") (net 4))
 (segment (start 96.87 101.29) (end 97 101.42) (width 0.2) (layer "B.Cu") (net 4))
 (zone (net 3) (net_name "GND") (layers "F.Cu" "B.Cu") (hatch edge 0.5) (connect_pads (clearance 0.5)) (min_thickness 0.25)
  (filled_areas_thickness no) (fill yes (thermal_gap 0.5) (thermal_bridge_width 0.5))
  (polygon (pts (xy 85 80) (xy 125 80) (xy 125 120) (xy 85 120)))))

